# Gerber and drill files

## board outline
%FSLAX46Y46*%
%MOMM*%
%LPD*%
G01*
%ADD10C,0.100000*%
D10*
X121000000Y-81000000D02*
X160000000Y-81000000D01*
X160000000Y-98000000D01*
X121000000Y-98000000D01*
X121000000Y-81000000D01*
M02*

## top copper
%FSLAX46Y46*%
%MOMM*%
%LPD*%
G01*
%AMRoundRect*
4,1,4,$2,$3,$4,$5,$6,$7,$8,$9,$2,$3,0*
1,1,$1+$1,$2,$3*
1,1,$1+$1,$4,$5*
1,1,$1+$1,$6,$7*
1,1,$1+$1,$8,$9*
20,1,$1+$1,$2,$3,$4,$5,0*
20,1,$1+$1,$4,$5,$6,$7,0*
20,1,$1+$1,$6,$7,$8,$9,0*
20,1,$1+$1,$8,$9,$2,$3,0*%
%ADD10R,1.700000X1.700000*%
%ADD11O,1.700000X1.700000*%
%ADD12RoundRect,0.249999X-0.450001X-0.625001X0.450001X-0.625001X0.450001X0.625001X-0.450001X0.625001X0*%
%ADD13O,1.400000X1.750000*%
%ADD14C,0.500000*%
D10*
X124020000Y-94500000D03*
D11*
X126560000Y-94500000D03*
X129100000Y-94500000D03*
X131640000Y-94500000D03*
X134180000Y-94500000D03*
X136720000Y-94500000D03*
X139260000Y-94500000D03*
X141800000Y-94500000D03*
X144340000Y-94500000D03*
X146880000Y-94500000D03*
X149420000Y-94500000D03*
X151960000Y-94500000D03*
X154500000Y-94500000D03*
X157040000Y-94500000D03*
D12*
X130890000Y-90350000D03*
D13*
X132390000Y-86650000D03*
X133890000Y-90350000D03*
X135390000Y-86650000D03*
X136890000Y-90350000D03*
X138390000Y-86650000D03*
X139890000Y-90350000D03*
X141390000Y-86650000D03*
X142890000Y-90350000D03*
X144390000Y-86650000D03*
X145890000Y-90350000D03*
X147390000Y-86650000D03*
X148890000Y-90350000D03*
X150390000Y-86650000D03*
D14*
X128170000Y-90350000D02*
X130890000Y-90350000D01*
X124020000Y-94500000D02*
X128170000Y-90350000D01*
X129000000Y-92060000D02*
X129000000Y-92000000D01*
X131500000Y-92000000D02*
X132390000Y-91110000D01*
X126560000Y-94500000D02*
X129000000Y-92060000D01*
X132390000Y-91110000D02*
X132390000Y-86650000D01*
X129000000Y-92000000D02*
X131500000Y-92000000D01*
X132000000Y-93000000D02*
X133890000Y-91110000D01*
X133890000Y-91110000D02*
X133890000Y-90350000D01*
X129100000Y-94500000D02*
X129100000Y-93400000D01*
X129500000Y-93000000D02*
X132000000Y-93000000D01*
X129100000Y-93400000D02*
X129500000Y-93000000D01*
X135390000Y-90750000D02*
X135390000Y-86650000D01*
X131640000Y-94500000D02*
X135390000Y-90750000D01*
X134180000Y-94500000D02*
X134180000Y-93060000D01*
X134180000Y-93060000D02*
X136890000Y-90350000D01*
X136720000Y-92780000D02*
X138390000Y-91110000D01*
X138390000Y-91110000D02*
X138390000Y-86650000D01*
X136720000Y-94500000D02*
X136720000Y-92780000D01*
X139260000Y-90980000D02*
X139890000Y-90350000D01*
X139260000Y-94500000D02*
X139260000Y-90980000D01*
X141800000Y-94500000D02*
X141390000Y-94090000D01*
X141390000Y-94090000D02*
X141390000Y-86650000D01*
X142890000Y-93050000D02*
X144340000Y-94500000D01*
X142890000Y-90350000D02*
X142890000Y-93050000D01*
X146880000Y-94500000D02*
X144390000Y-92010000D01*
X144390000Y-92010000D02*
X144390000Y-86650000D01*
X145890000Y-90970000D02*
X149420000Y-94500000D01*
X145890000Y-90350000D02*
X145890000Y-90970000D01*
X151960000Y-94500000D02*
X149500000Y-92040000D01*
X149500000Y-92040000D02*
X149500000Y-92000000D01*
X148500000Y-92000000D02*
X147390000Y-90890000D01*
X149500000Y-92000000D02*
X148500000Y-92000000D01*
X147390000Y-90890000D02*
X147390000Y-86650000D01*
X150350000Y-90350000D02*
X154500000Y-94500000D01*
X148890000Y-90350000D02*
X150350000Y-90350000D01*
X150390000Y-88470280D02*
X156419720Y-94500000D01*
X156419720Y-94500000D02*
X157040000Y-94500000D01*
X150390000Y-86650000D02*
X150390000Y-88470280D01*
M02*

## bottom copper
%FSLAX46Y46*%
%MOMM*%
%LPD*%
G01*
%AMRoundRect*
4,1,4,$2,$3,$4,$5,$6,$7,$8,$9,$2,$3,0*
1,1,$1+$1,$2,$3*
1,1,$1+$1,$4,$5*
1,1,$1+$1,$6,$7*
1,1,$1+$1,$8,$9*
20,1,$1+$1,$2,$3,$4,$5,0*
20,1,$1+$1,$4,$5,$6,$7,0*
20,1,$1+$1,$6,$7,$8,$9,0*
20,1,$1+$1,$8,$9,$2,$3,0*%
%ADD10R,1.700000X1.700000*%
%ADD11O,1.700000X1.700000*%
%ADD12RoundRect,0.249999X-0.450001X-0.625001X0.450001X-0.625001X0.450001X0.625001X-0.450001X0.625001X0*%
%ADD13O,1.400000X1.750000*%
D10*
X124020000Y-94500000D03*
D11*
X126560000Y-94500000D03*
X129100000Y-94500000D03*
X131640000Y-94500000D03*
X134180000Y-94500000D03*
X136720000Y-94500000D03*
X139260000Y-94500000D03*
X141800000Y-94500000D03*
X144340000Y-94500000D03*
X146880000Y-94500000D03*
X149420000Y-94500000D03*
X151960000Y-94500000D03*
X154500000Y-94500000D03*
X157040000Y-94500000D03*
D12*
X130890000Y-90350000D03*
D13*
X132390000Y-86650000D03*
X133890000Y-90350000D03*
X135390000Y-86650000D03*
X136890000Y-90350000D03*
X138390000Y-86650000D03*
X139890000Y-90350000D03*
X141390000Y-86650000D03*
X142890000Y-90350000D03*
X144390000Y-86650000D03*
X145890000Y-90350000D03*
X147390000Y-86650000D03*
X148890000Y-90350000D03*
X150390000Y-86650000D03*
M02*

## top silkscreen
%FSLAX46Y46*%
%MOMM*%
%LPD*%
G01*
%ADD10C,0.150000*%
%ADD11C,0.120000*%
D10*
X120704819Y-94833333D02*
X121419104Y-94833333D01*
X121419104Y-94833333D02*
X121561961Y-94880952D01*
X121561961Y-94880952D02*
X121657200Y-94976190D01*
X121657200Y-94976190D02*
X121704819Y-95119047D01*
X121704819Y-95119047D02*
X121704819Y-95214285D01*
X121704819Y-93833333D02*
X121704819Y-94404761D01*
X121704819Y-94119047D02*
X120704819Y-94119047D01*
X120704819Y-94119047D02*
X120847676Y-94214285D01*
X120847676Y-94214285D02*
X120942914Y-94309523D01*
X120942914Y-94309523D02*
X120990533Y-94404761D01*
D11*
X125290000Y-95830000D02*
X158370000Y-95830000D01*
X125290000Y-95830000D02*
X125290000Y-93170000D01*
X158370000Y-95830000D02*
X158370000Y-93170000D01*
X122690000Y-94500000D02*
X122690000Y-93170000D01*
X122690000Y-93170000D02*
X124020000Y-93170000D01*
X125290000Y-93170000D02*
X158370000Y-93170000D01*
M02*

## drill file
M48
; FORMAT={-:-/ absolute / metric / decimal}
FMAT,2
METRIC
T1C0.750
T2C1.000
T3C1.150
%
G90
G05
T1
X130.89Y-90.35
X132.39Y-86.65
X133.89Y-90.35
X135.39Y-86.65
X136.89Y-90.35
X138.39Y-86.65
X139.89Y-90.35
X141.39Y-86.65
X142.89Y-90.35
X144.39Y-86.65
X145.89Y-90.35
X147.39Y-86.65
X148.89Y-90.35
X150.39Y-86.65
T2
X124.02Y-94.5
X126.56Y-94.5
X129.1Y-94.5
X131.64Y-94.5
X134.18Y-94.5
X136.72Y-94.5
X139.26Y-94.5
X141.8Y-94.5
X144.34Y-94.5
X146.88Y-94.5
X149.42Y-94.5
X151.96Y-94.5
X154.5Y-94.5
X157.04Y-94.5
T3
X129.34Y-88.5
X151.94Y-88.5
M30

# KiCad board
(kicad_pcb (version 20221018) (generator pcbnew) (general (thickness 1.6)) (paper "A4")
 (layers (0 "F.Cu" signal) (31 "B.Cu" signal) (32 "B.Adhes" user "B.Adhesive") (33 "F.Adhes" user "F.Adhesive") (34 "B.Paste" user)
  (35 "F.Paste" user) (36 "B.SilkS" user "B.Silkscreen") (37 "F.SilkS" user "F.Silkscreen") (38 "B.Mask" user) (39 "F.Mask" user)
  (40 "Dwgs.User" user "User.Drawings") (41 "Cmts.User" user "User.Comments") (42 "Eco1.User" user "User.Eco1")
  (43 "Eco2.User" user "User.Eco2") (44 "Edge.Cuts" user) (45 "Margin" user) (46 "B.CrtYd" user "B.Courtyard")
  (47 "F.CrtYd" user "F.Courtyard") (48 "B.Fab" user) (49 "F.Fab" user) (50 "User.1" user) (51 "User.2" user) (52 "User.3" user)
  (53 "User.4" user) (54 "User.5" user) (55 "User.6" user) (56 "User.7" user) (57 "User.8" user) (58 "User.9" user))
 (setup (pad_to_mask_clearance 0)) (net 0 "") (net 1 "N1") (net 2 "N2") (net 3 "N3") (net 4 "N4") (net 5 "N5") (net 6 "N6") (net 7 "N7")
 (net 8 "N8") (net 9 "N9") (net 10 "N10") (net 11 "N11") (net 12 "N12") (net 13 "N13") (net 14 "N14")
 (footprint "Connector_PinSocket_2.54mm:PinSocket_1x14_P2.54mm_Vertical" (layer "F.Cu") (at 124.02 94.5 90)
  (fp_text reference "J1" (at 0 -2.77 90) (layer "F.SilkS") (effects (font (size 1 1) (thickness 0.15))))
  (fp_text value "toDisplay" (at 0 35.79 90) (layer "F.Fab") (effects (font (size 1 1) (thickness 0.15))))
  (fp_line (start -1.33 1.27) (end -1.33 34.35) (stroke (width 0.12) (type solid)) (layer "F.SilkS"))
  (fp_line (start -1.33 1.27) (end 1.33 1.27) (stroke (width 0.12) (type solid)) (layer "F.SilkS"))
  (fp_line (start -1.33 34.35) (end 1.33 34.35) (stroke (width 0.12) (type solid)) (layer "F.SilkS"))
  (fp_line (start 0 -1.33) (end 1.33 -1.33) (stroke (width 0.12) (type solid)) (layer "F.SilkS"))
  (fp_line (start 1.33 -1.33) (end 1.33 0) (stroke (width 0.12) (type solid)) (layer "F.SilkS"))
  (fp_line (start 1.33 1.27) (end 1.33 34.35) (stroke (width 0.12) (type solid)) (layer "F.SilkS"))
  (pad "1" thru_hole rect (at 0 0 90) (size 1.7 1.7) (drill 1) (layers "*.Cu" "*.Mask") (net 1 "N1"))
  (pad "2" thru_hole oval (at 0 2.54 90) (size 1.7 1.7) (drill 1) (layers "*.Cu" "*.Mask") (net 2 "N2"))
  (pad "3" thru_hole oval (at 0 5.08 90) (size 1.7 1.7) (drill 1) (layers "*.Cu" "*.Mask") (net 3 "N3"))
  (pad "4" thru_hole oval (at 0 7.62 90) (size 1.7 1.7) (drill 1) (layers "*.Cu" "*.Mask") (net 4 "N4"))
  (pad "5" thru_hole oval (at 0 10.16 90) (size 1.7 1.7) (drill 1) (layers "*.Cu" "*.Mask") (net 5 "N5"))
  (pad "6" thru_hole oval (at 0 12.7 90) (size 1.7 1.7) (drill 1) (layers "*.Cu" "*.Mask") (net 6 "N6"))
  (pad "7" thru_hole oval (at 0 15.24 90) (size 1.7 1.7) (drill 1) (layers "*.Cu" "*.Mask") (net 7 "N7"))
  (pad "8" thru_hole oval (at 0 17.78 90) (size 1.7 1.7) (drill 1) (layers "*.Cu" "*.Mask") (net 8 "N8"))
  (pad "9" thru_hole oval (at 0 20.32 90) (size 1.7 1.7) (drill 1) (layers "*.Cu" "*.Mask") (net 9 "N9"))
  (pad "10" thru_hole oval (at 0 22.86 90) (size 1.7 1.7) (drill 1) (layers "*.Cu" "*.Mask") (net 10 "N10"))
  (pad "11" thru_hole oval (at 0 25.4 90) (size 1.7 1.7) (drill 1) (layers "*.Cu" "*.Mask") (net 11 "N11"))
  (pad "12" thru_hole oval (at 0 27.94 90) (size 1.7 1.7) (drill 1) (layers "*.Cu" "*.Mask") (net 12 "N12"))
  (pad "13" thru_hole oval (at 0 30.48 90) (size 1.7 1.7) (drill 1) (layers "*.Cu" "*.Mask") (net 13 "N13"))
  (pad "14" thru_hole oval (at 0 33.02 90) (size 1.7 1.7) (drill 1) (layers "*.Cu" "*.Mask") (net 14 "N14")))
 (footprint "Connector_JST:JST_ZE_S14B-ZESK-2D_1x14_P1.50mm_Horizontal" (layer "B.Cu") (at 130.89 90.35)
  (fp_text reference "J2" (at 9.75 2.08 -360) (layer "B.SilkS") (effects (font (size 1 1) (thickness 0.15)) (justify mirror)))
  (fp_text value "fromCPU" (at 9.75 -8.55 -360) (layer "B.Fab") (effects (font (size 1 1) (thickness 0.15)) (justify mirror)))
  (pad "" np_thru_hole circle (at -1.55 -1.85) (size 1.15 1.15) (drill 1.15) (layers "*.Cu" "*.Mask"))
  (pad "" np_thru_hole circle (at 21.05 -1.85) (size 1.15 1.15) (drill 1.15) (layers "*.Cu" "*.Mask"))
  (pad "1" thru_hole roundrect (at 0 0) (size 1.4 1.75) (drill 0.75) (layers "*.Cu" "*.Mask") (roundrect_rratio 0.178571) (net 1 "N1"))
  (pad "2" thru_hole oval (at 1.5 -3.7) (size 1.4 1.75) (drill 0.75) (layers "*.Cu" "*.Mask") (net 2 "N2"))
  (pad "3" thru_hole oval (at 3 0) (size 1.4 1.75) (drill 0.75) (layers "*.Cu" "*.Mask") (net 3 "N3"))
  (pad "4" thru_hole oval (at 4.5 -3.7) (size 1.4 1.75) (drill 0.75) (layers "*.Cu" "*.Mask") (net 4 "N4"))
  (pad "5" thru_hole oval (at 6 0) (size 1.4 1.75) (drill 0.75) (layers "*.Cu" "*.Mask") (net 5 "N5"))
  (pad "6" thru_hole oval (at 7.5 -3.7) (size 1.4 1.75) (drill 0.75) (layers "*.Cu" "*.Mask") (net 6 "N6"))
  (pad "7" thru_hole oval (at 9 0) (size 1.4 1.75) (drill 0.75) (layers "*.Cu" "*.Mask") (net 7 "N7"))
  (pad "8" thru_hole oval (at 10.5 -3.7) (size 1.4 1.75) (drill 0.75) (layers "*.Cu" "*.Mask") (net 8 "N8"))
  (pad "9" thru_hole oval (at 12 0) (size 1.4 1.75) (drill 0.75) (layers "*.Cu" "*.Mask") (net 9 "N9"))
  (pad "10" thru_hole oval (at 13.5 -3.7) (size 1.4 1.75) (drill 0.75) (layers "*.Cu" "*.Mask") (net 10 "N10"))
  (pad "11" thru_hole oval (at 15 0) (size 1.4 1.75) (drill 0.75) (layers "*.Cu" "*.Mask") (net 11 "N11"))
  (pad "12" thru_hole oval (at 16.5 -3.7) (size 1.4 1.75) (drill 0.75) (layers "*.Cu" "*.Mask") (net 12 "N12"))
  (pad "13" thru_hole oval (at 18 0) (size 1.4 1.75) (drill 0.75) (layers "*.Cu" "*.Mask") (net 13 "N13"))
  (pad "14" thru_hole oval (at 19.5 -3.7) (size 1.4 1.75) (drill 0.75) (layers "*.Cu" "*.Mask") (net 14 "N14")))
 (gr_rect (start 121 81) (end 160 98) (stroke (width 0.1) (type default)) (fill none) (layer "Edge.Cuts"))
 (segment (start 128.17 90.35) (end 130.89 90.35) (width 0.5) (layer "F.Cu") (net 1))
 (segment (start 124.02 94.5) (end 128.17 90.35) (width 0.5) (layer "F.Cu") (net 1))
 (segment (start 129 92.06) (end 129 92) (width 0.5) (layer "F.Cu") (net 2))
 (segment (start 131.5 92) (end 132.39 91.11) (width 0.5) (layer "F.Cu") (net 2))
 (segment (start 126.56 94.5) (end 129 92.06) (width 0.5) (layer "F.Cu") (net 2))
 (segment (start 132.39 91.11) (end 132.39 86.65) (width 0.5) (layer "F.Cu") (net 2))
 (segment (start 129 92) (end 131.5 92) (width 0.5) (layer "F.Cu") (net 2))
 (segment (start 132 93) (end 133.89 91.11) (width 0.5) (layer "F.Cu") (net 3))
 (segment (start 133.89 91.11) (end 133.89 90.35) (width 0.5) (layer "F.Cu") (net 3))
 (segment (start 129.1 94.5) (end 129.1 93.4) (width 0.5) (layer "F.Cu") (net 3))
 (segment (start 129.5 93) (end 132 93) (width 0.5) (layer "F.Cu") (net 3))
 (segment (start 129.1 93.4) (end 129.5 93) (width 0.5) (layer "F.Cu") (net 3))
 (segment (start 135.39 90.75) (end 135.39 86.65) (width 0.5) (layer "F.Cu") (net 4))
 (segment (start 131.64 94.5) (end 135.39 90.75) (width 0.5) (layer "F.Cu") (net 4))
 (segment (start 134.18 94.5) (end 134.18 93.06) (width 0.5) (layer "F.Cu") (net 5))
 (segment (start 134.18 93.06) (end 136.89 90.35) (width 0.5) (layer "F.Cu") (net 5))
 (segment (start 136.72 92.78) (end 138.39 91.11) (width 0.5) (layer "F.Cu") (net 6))
 (segment (start 138.39 91.11) (end 138.39 86.65) (width 0.5) (layer "F.Cu") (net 6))
 (segment (start 136.72 94.5) (end 136.72 92.78) (width 0.5) (layer "F.Cu") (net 6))
 (segment (start 139.26 90.98) (end 139.89 90.35) (width 0.5) (layer "F.Cu") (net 7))
 (segment (start 139.26 94.5) (end 139.26 90.98) (width 0.5) (layer "F.Cu") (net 7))
 (segment (start 141.8 94.5) (end 141.39 94.09) (width 0.5) (layer "F.Cu") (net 8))
 (segment (start 141.39 94.09) (end 141.39 86.65) (width 0.5) (layer "F.Cu") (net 8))
 (segment (start 142.89 93.05) (end 144.34 94.5) (width 0.5) (layer "F.Cu") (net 9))
 (segment (start 142.89 90.35) (end 142.89 93.05) (width 0.5) (layer "F.Cu") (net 9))
 (segment (start 146.88 94.5) (end 144.39 92.01) (width 0.5) (layer "F.Cu") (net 10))
 (segment (start 144.39 92.01) (end 144.39 86.65) (width 0.5) (layer "F.Cu") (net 10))
 (segment (start 145.89 90.97) (end 149.42 94.5) (width 0.5) (layer "F.Cu") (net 11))
 (segment (start 145.89 90.35) (end 145.89 90.97) (width 0.5) (layer "F.Cu") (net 11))
 (segment (start 151.96 94.5) (end 149.5 92.04) (width 0.5) (layer "F.Cu") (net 12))
 (segment (start 149.5 92.04) (end 149.5 92) (width 0.5) (layer "F.Cu") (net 12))
 (segment (start 148.5 92) (end 147.39 90.89) (width 0.5) (layer "F.Cu") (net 12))
 (segment (start 149.5 92) (end 148.5 92) (width 0.5) (layer "F.Cu") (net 12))
 (segment (start 147.39 90.89) (end 147.39 86.65) (width 0.5) (layer "F.Cu") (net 12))
 (segment (start 150.35 90.35) (end 154.5 94.5) (width 0.5) (layer "F.Cu") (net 13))
 (segment (start 148.89 90.35) (end 150.35 90.35) (width 0.5) (layer "F.Cu") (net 13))
 (segment (start 150.39 88.47028) (end 156.41972 94.5) (width 0.5) (layer "F.Cu") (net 14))
 (segment (start 156.41972 94.5) (end 157.04 94.5) (width 0.5) (layer "F.Cu") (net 14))
 (segment (start 150.39 86.65) (end 150.39 88.47028) (width 0.5) (layer "F.Cu") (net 14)))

